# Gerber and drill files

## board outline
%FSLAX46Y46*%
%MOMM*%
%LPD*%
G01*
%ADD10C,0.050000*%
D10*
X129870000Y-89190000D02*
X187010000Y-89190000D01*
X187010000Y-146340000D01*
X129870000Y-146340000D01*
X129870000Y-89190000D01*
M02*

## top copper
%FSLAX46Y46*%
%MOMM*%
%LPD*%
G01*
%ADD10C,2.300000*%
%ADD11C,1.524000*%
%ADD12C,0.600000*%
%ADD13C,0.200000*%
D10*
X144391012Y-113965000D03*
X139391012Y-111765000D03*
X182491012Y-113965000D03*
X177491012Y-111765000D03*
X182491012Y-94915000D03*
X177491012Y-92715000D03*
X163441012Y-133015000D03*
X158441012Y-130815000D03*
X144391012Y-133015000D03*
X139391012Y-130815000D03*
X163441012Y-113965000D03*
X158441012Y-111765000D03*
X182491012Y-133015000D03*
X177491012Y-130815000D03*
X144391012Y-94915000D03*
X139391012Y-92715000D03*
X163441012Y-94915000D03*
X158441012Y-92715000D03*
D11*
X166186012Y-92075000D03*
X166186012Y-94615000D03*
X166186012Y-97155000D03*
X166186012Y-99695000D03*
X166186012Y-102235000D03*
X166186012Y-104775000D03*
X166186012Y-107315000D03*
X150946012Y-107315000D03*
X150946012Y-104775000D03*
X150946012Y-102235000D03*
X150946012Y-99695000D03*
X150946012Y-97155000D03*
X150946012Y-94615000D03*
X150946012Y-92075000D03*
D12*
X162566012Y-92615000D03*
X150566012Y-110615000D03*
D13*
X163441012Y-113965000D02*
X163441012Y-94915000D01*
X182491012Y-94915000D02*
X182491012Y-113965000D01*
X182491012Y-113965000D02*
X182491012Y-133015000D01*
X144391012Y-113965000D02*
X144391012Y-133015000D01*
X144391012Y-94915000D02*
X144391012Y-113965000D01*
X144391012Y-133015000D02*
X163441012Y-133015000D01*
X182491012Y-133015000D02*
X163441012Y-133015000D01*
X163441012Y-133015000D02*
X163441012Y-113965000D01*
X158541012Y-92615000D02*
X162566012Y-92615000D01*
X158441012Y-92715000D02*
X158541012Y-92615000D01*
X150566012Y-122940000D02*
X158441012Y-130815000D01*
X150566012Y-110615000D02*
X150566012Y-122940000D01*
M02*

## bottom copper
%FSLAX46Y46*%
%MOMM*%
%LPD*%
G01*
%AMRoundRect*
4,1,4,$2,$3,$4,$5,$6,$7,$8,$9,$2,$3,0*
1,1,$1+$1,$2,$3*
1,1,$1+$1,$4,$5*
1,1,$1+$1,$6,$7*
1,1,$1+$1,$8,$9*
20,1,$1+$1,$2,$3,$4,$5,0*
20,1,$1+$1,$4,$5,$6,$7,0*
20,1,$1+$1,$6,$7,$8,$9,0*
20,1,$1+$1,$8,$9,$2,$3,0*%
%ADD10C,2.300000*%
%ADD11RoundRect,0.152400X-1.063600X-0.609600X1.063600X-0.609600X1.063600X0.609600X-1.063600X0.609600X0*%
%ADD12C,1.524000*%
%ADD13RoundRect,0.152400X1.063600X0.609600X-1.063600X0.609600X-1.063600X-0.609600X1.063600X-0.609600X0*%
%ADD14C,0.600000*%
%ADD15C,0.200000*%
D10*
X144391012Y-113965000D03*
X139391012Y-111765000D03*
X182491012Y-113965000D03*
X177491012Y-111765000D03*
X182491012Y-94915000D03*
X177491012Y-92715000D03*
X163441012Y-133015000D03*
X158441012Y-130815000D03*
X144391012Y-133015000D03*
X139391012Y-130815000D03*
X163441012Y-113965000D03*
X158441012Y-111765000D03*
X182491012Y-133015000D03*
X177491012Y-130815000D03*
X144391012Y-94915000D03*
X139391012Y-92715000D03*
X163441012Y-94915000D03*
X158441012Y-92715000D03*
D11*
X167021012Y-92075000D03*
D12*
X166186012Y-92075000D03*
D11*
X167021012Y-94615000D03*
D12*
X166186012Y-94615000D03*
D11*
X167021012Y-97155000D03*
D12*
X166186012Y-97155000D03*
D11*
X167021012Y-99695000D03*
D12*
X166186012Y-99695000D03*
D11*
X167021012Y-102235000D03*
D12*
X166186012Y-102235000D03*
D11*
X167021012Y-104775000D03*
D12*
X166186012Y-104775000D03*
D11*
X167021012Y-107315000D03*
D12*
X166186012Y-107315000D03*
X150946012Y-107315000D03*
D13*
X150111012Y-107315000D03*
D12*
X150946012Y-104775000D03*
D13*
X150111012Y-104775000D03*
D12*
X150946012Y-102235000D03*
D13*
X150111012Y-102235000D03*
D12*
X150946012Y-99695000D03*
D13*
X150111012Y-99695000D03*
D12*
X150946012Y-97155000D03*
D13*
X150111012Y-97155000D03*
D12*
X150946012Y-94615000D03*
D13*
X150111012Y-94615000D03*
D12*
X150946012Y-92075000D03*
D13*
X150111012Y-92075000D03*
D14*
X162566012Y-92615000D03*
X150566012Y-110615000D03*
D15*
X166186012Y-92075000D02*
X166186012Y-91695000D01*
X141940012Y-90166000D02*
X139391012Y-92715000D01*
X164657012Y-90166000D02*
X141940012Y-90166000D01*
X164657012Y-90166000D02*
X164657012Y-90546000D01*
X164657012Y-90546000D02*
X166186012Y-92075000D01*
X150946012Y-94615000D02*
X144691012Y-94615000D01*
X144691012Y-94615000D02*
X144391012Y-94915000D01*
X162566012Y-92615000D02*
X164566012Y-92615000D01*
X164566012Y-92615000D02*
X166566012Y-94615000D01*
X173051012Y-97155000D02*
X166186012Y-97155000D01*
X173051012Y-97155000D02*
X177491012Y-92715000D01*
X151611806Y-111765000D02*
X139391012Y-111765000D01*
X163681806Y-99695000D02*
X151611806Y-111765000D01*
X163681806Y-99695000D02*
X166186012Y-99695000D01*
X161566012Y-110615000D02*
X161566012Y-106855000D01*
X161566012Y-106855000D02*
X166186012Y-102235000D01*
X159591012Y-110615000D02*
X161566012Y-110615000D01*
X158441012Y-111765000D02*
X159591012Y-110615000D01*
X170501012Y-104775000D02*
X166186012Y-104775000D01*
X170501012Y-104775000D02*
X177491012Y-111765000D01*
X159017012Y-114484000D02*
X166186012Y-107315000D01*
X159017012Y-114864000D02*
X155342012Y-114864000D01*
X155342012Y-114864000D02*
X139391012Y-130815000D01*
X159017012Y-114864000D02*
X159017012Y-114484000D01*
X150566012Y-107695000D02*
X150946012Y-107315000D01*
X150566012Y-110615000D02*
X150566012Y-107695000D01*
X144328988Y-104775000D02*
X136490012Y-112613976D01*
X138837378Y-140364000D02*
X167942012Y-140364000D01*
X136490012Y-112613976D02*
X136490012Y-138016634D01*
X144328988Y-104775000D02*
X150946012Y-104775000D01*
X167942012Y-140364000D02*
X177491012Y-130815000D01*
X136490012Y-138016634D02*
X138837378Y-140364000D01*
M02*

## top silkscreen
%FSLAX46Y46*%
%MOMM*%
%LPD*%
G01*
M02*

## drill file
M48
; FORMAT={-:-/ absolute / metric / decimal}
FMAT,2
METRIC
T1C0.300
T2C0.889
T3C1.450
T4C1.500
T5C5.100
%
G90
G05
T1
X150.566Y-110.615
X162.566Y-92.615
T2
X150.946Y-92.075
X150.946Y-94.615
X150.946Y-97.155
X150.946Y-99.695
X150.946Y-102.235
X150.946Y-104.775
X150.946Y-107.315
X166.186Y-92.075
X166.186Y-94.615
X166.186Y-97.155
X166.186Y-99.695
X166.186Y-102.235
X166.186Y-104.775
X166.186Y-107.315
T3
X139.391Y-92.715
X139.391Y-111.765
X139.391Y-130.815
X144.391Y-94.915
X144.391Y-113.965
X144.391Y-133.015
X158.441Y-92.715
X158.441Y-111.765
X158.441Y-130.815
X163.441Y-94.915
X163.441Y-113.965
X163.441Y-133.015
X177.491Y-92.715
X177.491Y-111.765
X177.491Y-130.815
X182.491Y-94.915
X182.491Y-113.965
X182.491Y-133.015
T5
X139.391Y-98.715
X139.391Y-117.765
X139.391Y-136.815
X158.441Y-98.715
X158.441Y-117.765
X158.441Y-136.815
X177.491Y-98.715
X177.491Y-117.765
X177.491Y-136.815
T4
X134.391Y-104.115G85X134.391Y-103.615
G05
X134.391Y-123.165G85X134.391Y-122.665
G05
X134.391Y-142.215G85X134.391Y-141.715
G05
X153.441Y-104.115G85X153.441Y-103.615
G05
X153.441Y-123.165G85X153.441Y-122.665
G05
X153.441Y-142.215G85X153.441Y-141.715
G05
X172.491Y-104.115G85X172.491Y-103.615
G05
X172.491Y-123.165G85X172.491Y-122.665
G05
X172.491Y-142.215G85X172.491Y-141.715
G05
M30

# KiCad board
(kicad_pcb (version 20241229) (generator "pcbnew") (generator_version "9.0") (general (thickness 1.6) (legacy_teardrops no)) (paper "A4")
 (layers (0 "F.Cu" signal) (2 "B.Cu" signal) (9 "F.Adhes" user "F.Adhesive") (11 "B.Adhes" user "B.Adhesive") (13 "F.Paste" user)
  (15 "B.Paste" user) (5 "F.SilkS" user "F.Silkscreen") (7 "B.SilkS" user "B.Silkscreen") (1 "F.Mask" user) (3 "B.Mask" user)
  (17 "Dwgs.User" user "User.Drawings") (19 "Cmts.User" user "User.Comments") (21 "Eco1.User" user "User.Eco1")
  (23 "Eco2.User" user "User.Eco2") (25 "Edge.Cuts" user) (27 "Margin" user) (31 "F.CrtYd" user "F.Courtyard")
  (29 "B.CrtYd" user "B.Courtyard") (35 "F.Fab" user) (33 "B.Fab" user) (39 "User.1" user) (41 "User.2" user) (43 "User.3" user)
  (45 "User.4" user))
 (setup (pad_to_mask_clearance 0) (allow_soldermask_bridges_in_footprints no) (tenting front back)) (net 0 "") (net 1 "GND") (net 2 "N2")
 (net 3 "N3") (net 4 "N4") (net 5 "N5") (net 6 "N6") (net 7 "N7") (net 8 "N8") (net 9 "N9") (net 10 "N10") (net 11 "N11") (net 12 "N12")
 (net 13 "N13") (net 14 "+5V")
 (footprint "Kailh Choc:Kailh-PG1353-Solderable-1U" (layer "F.Cu") (at 139.391012 117.765)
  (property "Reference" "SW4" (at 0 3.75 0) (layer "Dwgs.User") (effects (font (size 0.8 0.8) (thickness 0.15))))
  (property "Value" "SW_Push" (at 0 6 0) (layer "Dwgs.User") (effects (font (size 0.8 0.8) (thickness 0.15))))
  (pad "" np_thru_hole oval (at -5 5.15 180) (size 1.5 2) (drill oval 1.5 2) (layers "*.Cu" "*.Mask"))
  (pad "" np_thru_hole circle (at 0 0 180) (size 5 5) (drill 5.1) (layers "*.Cu" "*.Mask"))
  (pad "1" thru_hole circle (at 5 -3.8 180) (size 2.3 2.3) (drill 1.45) (layers "*.Cu" "B.Mask") (remove_unused_layers no) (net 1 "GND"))
  (pad "2" thru_hole circle (at 0 -6 180) (size 2.3 2.3) (drill 1.45) (layers "*.Cu" "B.Mask") (remove_unused_layers no) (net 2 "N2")))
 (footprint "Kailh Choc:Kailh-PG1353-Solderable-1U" (layer "F.Cu") (at 177.491012 117.765)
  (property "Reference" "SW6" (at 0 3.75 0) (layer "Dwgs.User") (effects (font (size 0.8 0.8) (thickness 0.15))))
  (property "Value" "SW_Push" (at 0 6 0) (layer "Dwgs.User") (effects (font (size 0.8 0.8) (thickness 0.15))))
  (pad "" np_thru_hole oval (at -5 5.15 180) (size 1.5 2) (drill oval 1.5 2) (layers "*.Cu" "*.Mask"))
  (pad "" np_thru_hole circle (at 0 0 180) (size 5 5) (drill 5.1) (layers "*.Cu" "*.Mask"))
  (pad "1" thru_hole circle (at 5 -3.8 180) (size 2.3 2.3) (drill 1.45) (layers "*.Cu" "B.Mask") (remove_unused_layers no) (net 1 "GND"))
  (pad "2" thru_hole circle (at 0 -6 180) (size 2.3 2.3) (drill 1.45) (layers "*.Cu" "B.Mask") (remove_unused_layers no) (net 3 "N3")))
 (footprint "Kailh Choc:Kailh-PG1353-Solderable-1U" (layer "F.Cu") (at 177.491012 98.715)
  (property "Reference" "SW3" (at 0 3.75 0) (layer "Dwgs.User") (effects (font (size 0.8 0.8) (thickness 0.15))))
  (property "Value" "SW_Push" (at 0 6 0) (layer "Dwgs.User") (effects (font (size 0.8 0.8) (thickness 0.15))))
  (pad "" np_thru_hole oval (at -5 5.15 180) (size 1.5 2) (drill oval 1.5 2) (layers "*.Cu" "*.Mask"))
  (pad "" np_thru_hole circle (at 0 0 180) (size 5 5) (drill 5.1) (layers "*.Cu" "*.Mask"))
  (pad "1" thru_hole circle (at 5 -3.8 180) (size 2.3 2.3) (drill 1.45) (layers "*.Cu" "B.Mask") (remove_unused_layers no) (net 1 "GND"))
  (pad "2" thru_hole circle (at 0 -6 180) (size 2.3 2.3) (drill 1.45) (layers "*.Cu" "B.Mask") (remove_unused_layers no) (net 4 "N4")))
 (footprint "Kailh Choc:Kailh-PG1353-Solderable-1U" (layer "F.Cu") (at 158.441012 136.815)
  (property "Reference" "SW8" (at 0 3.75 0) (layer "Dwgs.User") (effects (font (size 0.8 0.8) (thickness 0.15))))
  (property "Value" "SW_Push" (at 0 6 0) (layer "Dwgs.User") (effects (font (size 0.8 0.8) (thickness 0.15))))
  (pad "" np_thru_hole oval (at -5 5.15 180) (size 1.5 2) (drill oval 1.5 2) (layers "*.Cu" "*.Mask"))
  (pad "" np_thru_hole circle (at 0 0 180) (size 5 5) (drill 5.1) (layers "*.Cu" "*.Mask"))
  (pad "1" thru_hole circle (at 5 -3.8 180) (size 2.3 2.3) (drill 1.45) (layers "*.Cu" "B.Mask") (remove_unused_layers no) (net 1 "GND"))
  (pad "2" thru_hole circle (at 0 -6 180) (size 2.3 2.3) (drill 1.45) (layers "*.Cu" "B.Mask") (remove_unused_layers no) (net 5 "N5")))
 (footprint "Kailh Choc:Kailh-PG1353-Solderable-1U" (layer "F.Cu") (at 139.391012 136.815)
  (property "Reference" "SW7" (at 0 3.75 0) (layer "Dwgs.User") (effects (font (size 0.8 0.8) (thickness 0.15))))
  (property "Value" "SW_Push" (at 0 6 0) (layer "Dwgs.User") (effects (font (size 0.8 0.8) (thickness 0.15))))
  (pad "" np_thru_hole oval (at -5 5.15 180) (size 1.5 2) (drill oval 1.5 2) (layers "*.Cu" "*.Mask"))
  (pad "" np_thru_hole circle (at 0 0 180) (size 5 5) (drill 5.1) (layers "*.Cu" "*.Mask"))
  (pad "1" thru_hole circle (at 5 -3.8 180) (size 2.3 2.3) (drill 1.45) (layers "*.Cu" "B.Mask") (remove_unused_layers no) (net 1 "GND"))
  (pad "2" thru_hole circle (at 0 -6 180) (size 2.3 2.3) (drill 1.45) (layers "*.Cu" "B.Mask") (remove_unused_layers no) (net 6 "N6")))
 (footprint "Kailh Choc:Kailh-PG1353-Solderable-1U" (layer "F.Cu") (at 158.441012 117.765)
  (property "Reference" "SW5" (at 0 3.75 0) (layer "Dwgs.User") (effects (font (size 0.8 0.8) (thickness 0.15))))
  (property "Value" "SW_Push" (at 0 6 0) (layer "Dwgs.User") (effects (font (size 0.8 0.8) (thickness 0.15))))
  (pad "" np_thru_hole oval (at -5 5.15 180) (size 1.5 2) (drill oval 1.5 2) (layers "*.Cu" "*.Mask"))
  (pad "" np_thru_hole circle (at 0 0 180) (size 5 5) (drill 5.1) (layers "*.Cu" "*.Mask"))
  (pad "1" thru_hole circle (at 5 -3.8 180) (size 2.3 2.3) (drill 1.45) (layers "*.Cu" "B.Mask") (remove_unused_layers no) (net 1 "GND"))
  (pad "2" thru_hole circle (at 0 -6 180) (size 2.3 2.3) (drill 1.45) (layers "*.Cu" "B.Mask") (remove_unused_layers no) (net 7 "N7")))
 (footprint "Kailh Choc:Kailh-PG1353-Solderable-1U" (layer "F.Cu") (at 177.491012 136.815)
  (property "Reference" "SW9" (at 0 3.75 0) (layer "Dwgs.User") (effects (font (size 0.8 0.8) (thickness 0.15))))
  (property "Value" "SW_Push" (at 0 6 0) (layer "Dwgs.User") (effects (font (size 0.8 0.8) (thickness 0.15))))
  (pad "" np_thru_hole oval (at -5 5.15 180) (size 1.5 2) (drill oval 1.5 2) (layers "*.Cu" "*.Mask"))
  (pad "" np_thru_hole circle (at 0 0 180) (size 5 5) (drill 5.1) (layers "*.Cu" "*.Mask"))
  (pad "1" thru_hole circle (at 5 -3.8 180) (size 2.3 2.3) (drill 1.45) (layers "*.Cu" "B.Mask") (remove_unused_layers no) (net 1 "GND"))
  (pad "2" thru_hole circle (at 0 -6 180) (size 2.3 2.3) (drill 1.45) (layers "*.Cu" "B.Mask") (remove_unused_layers no) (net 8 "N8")))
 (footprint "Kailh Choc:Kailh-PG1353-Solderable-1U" (layer "F.Cu") (at 139.391012 98.715)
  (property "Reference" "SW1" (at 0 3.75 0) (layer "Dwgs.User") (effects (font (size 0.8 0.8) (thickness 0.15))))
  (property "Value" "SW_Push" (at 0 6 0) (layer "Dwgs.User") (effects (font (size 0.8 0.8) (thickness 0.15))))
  (pad "" np_thru_hole oval (at -5 5.15 180) (size 1.5 2) (drill oval 1.5 2) (layers "*.Cu" "*.Mask"))
  (pad "" np_thru_hole circle (at 0 0 180) (size 5 5) (drill 5.1) (layers "*.Cu" "*.Mask"))
  (pad "1" thru_hole circle (at 5 -3.8 180) (size 2.3 2.3) (drill 1.45) (layers "*.Cu" "B.Mask") (remove_unused_layers no) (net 1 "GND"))
  (pad "2" thru_hole circle (at 0 -6 180) (size 2.3 2.3) (drill 1.45) (layers "*.Cu" "B.Mask") (remove_unused_layers no) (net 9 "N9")))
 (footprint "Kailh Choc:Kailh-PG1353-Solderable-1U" (layer "F.Cu") (at 158.441012 98.715)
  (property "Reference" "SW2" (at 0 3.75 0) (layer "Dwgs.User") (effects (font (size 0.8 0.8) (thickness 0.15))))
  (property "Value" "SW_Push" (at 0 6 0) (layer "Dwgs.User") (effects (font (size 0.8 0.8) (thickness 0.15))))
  (pad "" np_thru_hole oval (at -5 5.15 180) (size 1.5 2) (drill oval 1.5 2) (layers "*.Cu" "*.Mask"))
  (pad "" np_thru_hole circle (at 0 0 180) (size 5 5) (drill 5.1) (layers "*.Cu" "*.Mask"))
  (pad "1" thru_hole circle (at 5 -3.8 180) (size 2.3 2.3) (drill 1.45) (layers "*.Cu" "B.Mask") (remove_unused_layers no) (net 1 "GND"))
  (pad "2" thru_hole circle (at 0 -6 180) (size 2.3 2.3) (drill 1.45) (layers "*.Cu" "B.Mask") (remove_unused_layers no) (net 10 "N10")))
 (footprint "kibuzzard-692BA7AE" (layer "B.Cu") (at 134.1 91.54 180)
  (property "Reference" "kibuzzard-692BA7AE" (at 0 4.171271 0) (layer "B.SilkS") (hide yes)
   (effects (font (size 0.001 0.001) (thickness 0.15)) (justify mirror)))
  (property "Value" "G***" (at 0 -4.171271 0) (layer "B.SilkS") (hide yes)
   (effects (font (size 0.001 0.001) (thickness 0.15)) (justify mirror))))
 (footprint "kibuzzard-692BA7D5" (layer "B.Cu") (at 135.01 93.3 180)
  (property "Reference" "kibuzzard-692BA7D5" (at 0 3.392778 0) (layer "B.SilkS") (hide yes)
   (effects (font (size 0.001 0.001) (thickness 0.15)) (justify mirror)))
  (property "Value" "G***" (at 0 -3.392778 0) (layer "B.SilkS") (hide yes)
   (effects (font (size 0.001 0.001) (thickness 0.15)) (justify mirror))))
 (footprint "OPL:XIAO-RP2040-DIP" (layer "B.Cu") (at 158.566012 99.695 180)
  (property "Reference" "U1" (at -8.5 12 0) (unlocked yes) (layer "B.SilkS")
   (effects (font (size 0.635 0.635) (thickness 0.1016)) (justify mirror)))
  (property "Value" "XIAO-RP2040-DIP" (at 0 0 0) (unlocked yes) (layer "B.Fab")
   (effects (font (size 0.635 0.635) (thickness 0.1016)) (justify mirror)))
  (pad "1" smd roundrect (at -8.455 7.62) (size 2.432 1.524) (layers "B.Cu" "B.Mask") (roundrect_rratio 0.1) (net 9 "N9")
   (thermal_bridge_angle 45))
  (pad "1" thru_hole circle (at -7.62 7.62) (size 1.524 1.524) (drill 0.889) (layers "*.Cu" "*.Mask") (remove_unused_layers no) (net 9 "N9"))
  (pad "2" smd roundrect (at -8.455 5.08) (size 2.432 1.524) (layers "B.Cu" "B.Mask") (roundrect_rratio 0.1) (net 10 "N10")
   (thermal_bridge_angle 45))
  (pad "2" thru_hole circle (at -7.62 5.08) (size 1.524 1.524) (drill 0.889) (layers "*.Cu" "*.Mask") (remove_unused_layers no)
   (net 10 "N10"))
  (pad "3" smd roundrect (at -8.455 2.54) (size 2.432 1.524) (layers "B.Cu" "B.Mask") (roundrect_rratio 0.1) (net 4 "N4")
   (thermal_bridge_angle 45))
  (pad "3" thru_hole circle (at -7.62 2.54) (size 1.524 1.524) (drill 0.889) (layers "*.Cu" "*.Mask") (remove_unused_layers no) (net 4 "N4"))
  (pad "4" smd roundrect (at -8.455 0) (size 2.432 1.524) (layers "B.Cu" "B.Mask") (roundrect_rratio 0.1) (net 2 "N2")
   (thermal_bridge_angle 45))
  (pad "4" thru_hole circle (at -7.62 0) (size 1.524 1.524) (drill 0.889) (layers "*.Cu" "*.Mask") (remove_unused_layers no) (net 2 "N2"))
  (pad "5" smd roundrect (at -8.455 -2.54) (size 2.432 1.524) (layers "B.Cu" "B.Mask") (roundrect_rratio 0.1) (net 7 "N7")
   (thermal_bridge_angle 45))
  (pad "5" thru_hole circle (at -7.62 -2.54) (size 1.524 1.524) (drill 0.889) (layers "*.Cu" "*.Mask") (remove_unused_layers no)
   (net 7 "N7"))
  (pad "6" smd roundrect (at -8.455 -5.08) (size 2.432 1.524) (layers "B.Cu" "B.Mask") (roundrect_rratio 0.1) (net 3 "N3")
   (thermal_bridge_angle 45))
  (pad "6" thru_hole circle (at -7.62 -5.08) (size 1.524 1.524) (drill 0.889) (layers "*.Cu" "*.Mask") (remove_unused_layers no)
   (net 3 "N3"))
  (pad "7" smd roundrect (at -8.455 -7.62) (size 2.432 1.524) (layers "B.Cu" "B.Mask") (roundrect_rratio 0.1) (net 6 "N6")
   (thermal_bridge_angle 45))
  (pad "7" thru_hole circle (at -7.62 -7.62) (size 1.524 1.524) (drill 0.889) (layers "*.Cu" "*.Mask") (remove_unused_layers no)
   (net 6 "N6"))
  (pad "8" thru_hole circle (at 7.62 -7.62 180) (size 1.524 1.524) (drill 0.889) (layers "*.Cu" "*.Mask") (remove_unused_layers no)
   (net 5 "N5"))
  (pad "8" smd roundrect (at 8.455 -7.62 180) (size 2.432 1.524) (layers "B.Cu" "B.Mask") (roundrect_rratio 0.1) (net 5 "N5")
   (thermal_bridge_angle 45))
  (pad "9" thru_hole circle (at 7.62 -5.08 180) (size 1.524 1.524) (drill 0.889) (layers "*.Cu" "*.Mask") (remove_unused_layers no)
   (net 8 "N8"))
  (pad "9" smd roundrect (at 8.455 -5.08 180) (size 2.432 1.524) (layers "B.Cu" "B.Mask") (roundrect_rratio 0.1) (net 8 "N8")
   (thermal_bridge_angle 45))
  (pad "10" thru_hole circle (at 7.62 -2.54 180) (size 1.524 1.524) (drill 0.889) (layers "*.Cu" "*.Mask") (remove_unused_layers no)
   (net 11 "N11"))
  (pad "10" smd roundrect (at 8.455 -2.54 180) (size 2.432 1.524) (layers "B.Cu" "B.Mask") (roundrect_rratio 0.1) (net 11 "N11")
   (thermal_bridge_angle 45))
  (pad "11" thru_hole circle (at 7.62 0 180) (size 1.524 1.524) (drill 0.889) (layers "*.Cu" "*.Mask") (remove_unused_layers no)
   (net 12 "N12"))
  (pad "11" smd roundrect (at 8.455 0 180) (size 2.432 1.524) (layers "B.Cu" "B.Mask") (roundrect_rratio 0.1) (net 12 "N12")
   (thermal_bridge_angle 45))
  (pad "12" thru_hole circle (at 7.62 2.54 180) (size 1.524 1.524) (drill 0.889) (layers "*.Cu" "*.Mask") (remove_unused_layers no)
   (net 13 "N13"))
  (pad "12" smd roundrect (at 8.455 2.54 180) (size 2.432 1.524) (layers "B.Cu" "B.Mask") (roundrect_rratio 0.1) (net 13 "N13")
   (thermal_bridge_angle 45))
  (pad "13" thru_hole circle (at 7.62 5.08 180) (size 1.524 1.524) (drill 0.889) (layers "*.Cu" "*.Mask") (remove_unused_layers no)
   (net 1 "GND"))
  (pad "13" smd roundrect (at 8.455 5.08 180) (size 2.432 1.524) (layers "B.Cu" "B.Mask") (roundrect_rratio 0.1) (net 1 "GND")
   (thermal_bridge_angle 45))
  (pad "14" thru_hole circle (at 7.62 7.62 180) (size 1.524 1.524) (drill 0.889) (layers "*.Cu" "*.Mask") (remove_unused_layers no)
   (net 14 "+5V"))
  (pad "14" smd roundrect (at 8.455 7.62 180) (size 2.432 1.524) (layers "B.Cu" "B.Mask") (roundrect_rratio 0.1) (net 14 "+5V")
   (thermal_bridge_angle 45)))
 (gr_rect (start 129.87 89.19) (end 187.01 146.34) (stroke (width 0.05) (type default)) (fill no) (layer "Edge.Cuts"))
 (segment (start 166.186012 92.075) (end 166.186012 91.695) (width 0.2) (layer "B.Cu") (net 9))
 (segment (start 141.940012 90.166) (end 139.391012 92.715) (width 0.2) (layer "B.Cu") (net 9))
 (segment (start 164.657012 90.166) (end 141.940012 90.166) (width 0.2) (layer "B.Cu") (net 9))
 (segment (start 164.657012 90.166) (end 164.657012 90.546) (width 0.2) (layer "B.Cu") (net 9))
 (segment (start 164.657012 90.546) (end 166.186012 92.075) (width 0.2) (layer "B.Cu") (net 9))
 (segment (start 163.441012 113.965) (end 163.441012 94.915) (width 0.2) (layer "F.Cu") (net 1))
 (segment (start 182.491012 94.915) (end 182.491012 113.965) (width 0.2) (layer "F.Cu") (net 1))
 (segment (start 182.491012 113.965) (end 182.491012 133.015) (width 0.2) (layer "F.Cu") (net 1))
 (segment (start 144.391012 113.965) (end 144.391012 133.015) (width 0.2) (layer "F.Cu") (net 1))
 (segment (start 144.391012 94.915) (end 144.391012 113.965) (width 0.2) (layer "F.Cu") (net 1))
 (segment (start 144.391012 133.015) (end 163.441012 133.015) (width 0.2) (layer "F.Cu") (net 1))
 (segment (start 182.491012 133.015) (end 163.441012 133.015) (width 0.2) (layer "F.Cu") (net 1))
 (segment (start 163.441012 133.015) (end 163.441012 113.965) (width 0.2) (layer "F.Cu") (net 1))
 (segment (start 150.946012 94.615) (end 144.691012 94.615) (width 0.2) (layer "B.Cu") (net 1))
 (segment (start 144.691012 94.615) (end 144.391012 94.915) (width 0.2) (layer "B.Cu") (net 1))
 (segment (start 158.541012 92.615) (end 162.566012 92.615) (width 0.2) (layer "F.Cu") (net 10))
 (segment (start 158.441012 92.715) (end 158.541012 92.615) (width 0.2) (layer "F.Cu") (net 10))
 (via (at 162.566012 92.615) (size 0.6) (drill 0.3) (layers "F.Cu" "B.Cu") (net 10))
 (segment (start 162.566012 92.615) (end 164.566012 92.615) (width 0.2) (layer "B.Cu") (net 10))
 (segment (start 164.566012 92.615) (end 166.566012 94.615) (width 0.2) (layer "B.Cu") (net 10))
 (segment (start 173.051012 97.155) (end 166.186012 97.155) (width 0.2) (layer "B.Cu") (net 4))
 (segment (start 173.051012 97.155) (end 177.491012 92.715) (width 0.2) (layer "B.Cu") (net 4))
 (segment (start 151.611806 111.765) (end 139.391012 111.765) (width 0.2) (layer "B.Cu") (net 2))
 (segment (start 163.681806 99.695) (end 151.611806 111.765) (width 0.2) (layer "B.Cu") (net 2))
 (segment (start 163.681806 99.695) (end 166.186012 99.695) (width 0.2) (layer "B.Cu") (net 2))
 (segment (start 161.566012 110.615) (end 161.566012 106.855) (width 0.2) (layer "B.Cu") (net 7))
 (segment (start 161.566012 106.855) (end 166.186012 102.235) (width 0.2) (layer "B.Cu") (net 7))
 (segment (start 159.591012 110.615) (end 161.566012 110.615) (width 0.2) (layer "B.Cu") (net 7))
 (segment (start 158.441012 111.765) (end 159.591012 110.615) (width 0.2) (layer "B.Cu") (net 7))
 (segment (start 170.501012 104.775) (end 166.186012 104.775) (width 0.2) (layer "B.Cu") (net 3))
 (segment (start 170.501012 104.775) (end 177.491012 111.765) (width 0.2) (layer "B.Cu") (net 3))
 (segment (start 159.017012 114.484) (end 166.186012 107.315) (width 0.2) (layer "B.Cu") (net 6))
 (segment (start 159.017012 114.864) (end 155.342012 114.864) (width 0.2) (layer "B.Cu") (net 6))
 (segment (start 155.342012 114.864) (end 139.391012 130.815) (width 0.2) (layer "B.Cu") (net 6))
 (segment (start 159.017012 114.864) (end 159.017012 114.484) (width 0.2) (layer "B.Cu") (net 6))
 (segment (start 150.566012 122.94) (end 158.441012 130.815) (width 0.2) (layer "F.Cu") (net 5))
 (segment (start 150.566012 110.615) (end 150.566012 122.94) (width 0.2) (layer "F.Cu") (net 5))
 (via (at 150.566012 110.615) (size 0.6) (drill 0.3) (layers "F.Cu" "B.Cu") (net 5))
 (segment (start 150.566012 107.695) (end 150.946012 107.315) (width 0.2) (layer "B.Cu") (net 5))
 (segment (start 150.566012 110.615) (end 150.566012 107.695) (width 0.2) (layer "B.Cu") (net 5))
 (segment (start 144.328988 104.775) (end 136.490012 112.613976) (width 0.2) (layer "B.Cu") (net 8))
 (segment (start 138.837378 140.364) (end 167.942012 140.364) (width 0.2) (layer "B.Cu") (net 8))
 (segment (start 136.490012 112.613976) (end 136.490012 138.016634) (width 0.2) (layer "B.Cu") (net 8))
 (segment (start 144.328988 104.775) (end 150.946012 104.775) (width 0.2) (layer "B.Cu") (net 8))
 (segment (start 167.942012 140.364) (end 177.491012 130.815) (width 0.2) (layer "B.Cu") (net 8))
 (segment (start 136.490012 138.016634) (end 138.837378 140.364) (width 0.2) (layer "B.Cu") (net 8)))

